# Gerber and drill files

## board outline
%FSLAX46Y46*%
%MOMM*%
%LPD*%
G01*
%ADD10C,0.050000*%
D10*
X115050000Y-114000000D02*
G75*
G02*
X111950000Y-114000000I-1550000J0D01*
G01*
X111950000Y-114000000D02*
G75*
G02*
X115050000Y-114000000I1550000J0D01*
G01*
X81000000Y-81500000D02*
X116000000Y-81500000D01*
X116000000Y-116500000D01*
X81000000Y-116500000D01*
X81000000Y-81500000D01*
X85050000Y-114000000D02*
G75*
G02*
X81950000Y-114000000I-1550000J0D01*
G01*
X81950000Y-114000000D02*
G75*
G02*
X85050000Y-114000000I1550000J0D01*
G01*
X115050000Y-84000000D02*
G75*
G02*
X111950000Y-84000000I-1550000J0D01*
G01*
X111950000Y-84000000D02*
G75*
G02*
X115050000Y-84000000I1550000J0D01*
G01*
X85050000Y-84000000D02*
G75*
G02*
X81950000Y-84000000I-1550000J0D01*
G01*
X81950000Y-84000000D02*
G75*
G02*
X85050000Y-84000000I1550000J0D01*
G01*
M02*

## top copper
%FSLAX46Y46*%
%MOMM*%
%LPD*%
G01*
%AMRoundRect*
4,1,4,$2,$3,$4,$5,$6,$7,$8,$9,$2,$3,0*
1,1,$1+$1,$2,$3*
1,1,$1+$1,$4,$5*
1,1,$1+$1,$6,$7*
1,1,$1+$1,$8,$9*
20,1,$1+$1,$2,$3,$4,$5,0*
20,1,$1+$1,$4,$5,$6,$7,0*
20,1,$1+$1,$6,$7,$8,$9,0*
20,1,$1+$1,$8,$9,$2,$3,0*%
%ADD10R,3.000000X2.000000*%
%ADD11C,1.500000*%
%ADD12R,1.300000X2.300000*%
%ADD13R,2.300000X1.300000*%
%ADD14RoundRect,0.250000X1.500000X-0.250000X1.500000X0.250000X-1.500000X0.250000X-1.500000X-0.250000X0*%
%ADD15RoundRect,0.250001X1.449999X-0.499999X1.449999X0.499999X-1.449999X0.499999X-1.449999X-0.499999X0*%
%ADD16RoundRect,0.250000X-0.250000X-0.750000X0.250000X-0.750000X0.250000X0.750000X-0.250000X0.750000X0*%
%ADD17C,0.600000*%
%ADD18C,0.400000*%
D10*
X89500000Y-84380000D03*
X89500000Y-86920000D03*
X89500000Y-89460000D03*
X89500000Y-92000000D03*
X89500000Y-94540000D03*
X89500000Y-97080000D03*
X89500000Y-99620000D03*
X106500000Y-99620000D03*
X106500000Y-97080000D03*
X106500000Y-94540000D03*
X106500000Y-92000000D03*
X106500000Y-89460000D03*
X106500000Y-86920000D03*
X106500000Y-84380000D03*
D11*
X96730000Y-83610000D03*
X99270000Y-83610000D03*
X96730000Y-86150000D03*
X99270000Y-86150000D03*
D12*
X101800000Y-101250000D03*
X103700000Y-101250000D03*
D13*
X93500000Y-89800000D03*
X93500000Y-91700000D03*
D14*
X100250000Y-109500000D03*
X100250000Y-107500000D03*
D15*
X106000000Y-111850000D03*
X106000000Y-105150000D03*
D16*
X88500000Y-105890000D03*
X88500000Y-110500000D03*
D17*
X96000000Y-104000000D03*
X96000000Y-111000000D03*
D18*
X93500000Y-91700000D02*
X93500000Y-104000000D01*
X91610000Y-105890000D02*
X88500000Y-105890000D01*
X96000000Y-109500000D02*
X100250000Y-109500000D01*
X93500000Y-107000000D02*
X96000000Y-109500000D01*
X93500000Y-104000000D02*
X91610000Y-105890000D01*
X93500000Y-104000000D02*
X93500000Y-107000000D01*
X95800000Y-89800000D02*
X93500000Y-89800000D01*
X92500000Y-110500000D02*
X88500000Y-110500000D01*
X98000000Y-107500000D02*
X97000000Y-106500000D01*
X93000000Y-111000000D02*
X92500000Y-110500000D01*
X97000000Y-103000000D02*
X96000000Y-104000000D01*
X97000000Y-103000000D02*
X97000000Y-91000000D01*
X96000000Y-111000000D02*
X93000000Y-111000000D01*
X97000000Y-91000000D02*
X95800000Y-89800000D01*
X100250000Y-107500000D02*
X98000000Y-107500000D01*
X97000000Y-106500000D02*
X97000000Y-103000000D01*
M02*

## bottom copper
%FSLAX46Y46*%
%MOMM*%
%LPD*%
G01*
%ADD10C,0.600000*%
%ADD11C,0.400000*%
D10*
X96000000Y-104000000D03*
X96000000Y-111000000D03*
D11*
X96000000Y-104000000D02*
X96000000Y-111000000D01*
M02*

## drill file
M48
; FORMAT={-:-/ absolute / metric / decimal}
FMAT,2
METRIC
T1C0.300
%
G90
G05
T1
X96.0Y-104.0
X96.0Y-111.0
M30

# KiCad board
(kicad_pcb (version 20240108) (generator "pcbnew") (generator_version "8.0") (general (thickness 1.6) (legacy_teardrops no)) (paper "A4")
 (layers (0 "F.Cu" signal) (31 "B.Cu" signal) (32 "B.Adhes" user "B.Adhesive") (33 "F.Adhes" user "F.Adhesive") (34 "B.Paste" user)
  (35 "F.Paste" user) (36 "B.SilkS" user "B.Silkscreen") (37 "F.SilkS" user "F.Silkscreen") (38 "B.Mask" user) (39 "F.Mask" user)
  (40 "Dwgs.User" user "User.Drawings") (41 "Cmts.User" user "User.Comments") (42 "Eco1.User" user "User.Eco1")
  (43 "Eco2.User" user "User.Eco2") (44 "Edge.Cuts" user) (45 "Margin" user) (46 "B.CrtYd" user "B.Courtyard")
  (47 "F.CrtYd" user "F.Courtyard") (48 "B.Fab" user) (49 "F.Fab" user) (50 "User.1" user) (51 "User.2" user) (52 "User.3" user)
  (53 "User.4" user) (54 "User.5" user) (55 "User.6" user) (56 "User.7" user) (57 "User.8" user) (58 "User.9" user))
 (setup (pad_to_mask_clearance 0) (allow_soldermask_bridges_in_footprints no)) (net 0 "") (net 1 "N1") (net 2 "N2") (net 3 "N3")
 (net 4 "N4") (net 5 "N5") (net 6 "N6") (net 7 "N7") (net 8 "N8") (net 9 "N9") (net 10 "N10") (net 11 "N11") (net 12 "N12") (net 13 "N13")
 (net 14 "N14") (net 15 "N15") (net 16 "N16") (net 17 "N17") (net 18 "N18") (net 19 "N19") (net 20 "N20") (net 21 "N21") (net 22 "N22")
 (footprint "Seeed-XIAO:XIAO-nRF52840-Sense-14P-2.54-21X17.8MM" (layer "F.Cu") (at 98 92)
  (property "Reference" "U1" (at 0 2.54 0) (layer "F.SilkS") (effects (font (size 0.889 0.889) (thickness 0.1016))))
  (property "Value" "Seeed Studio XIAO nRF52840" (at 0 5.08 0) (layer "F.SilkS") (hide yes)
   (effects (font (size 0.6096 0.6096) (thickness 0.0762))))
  (pad "1" smd rect (at -8.5 -7.62) (size 3 2) (layers "F.Cu" "F.Paste" "F.Mask") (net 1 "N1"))
  (pad "2" smd rect (at -8.5 -5.08) (size 3 2) (layers "F.Cu" "F.Paste" "F.Mask") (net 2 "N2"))
  (pad "3" smd rect (at -8.5 -2.54) (size 3 2) (layers "F.Cu" "F.Paste" "F.Mask") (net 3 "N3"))
  (pad "4" smd rect (at -8.5 0) (size 3 2) (layers "F.Cu" "F.Paste" "F.Mask") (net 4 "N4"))
  (pad "5" smd rect (at -8.5 2.54) (size 3 2) (layers "F.Cu" "F.Paste" "F.Mask") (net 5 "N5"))
  (pad "6" smd rect (at -8.5 5.08 180) (size 3 2) (layers "F.Cu" "F.Paste" "F.Mask") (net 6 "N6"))
  (pad "7" smd rect (at -8.5 7.62) (size 3 2) (layers "F.Cu" "F.Paste" "F.Mask") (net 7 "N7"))
  (pad "8" smd rect (at 8.5 7.62) (size 3 2) (layers "F.Cu" "F.Paste" "F.Mask") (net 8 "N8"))
  (pad "9" smd rect (at 8.5 5.08) (size 3 2) (layers "F.Cu" "F.Paste" "F.Mask") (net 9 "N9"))
  (pad "10" smd rect (at 8.5 2.54) (size 3 2) (layers "F.Cu" "F.Paste" "F.Mask") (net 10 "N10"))
  (pad "11" smd rect (at 8.5 0) (size 3 2) (layers "F.Cu" "F.Paste" "F.Mask") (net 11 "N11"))
  (pad "12" smd rect (at 8.5 -2.54) (size 3 2) (layers "F.Cu" "F.Paste" "F.Mask") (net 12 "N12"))
  (pad "13" smd rect (at 8.5 -5.08) (size 3 2) (layers "F.Cu" "F.Paste" "F.Mask") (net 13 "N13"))
  (pad "14" smd rect (at 8.5 -7.62) (size 3 2) (layers "F.Cu" "F.Paste" "F.Mask") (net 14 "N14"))
  (pad "15" smd circle (at -1.27 -8.39 90) (size 1.5 1.5) (layers "F.Cu" "F.Paste" "F.Mask") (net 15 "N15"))
  (pad "16" smd circle (at 1.27 -8.39 90) (size 1.5 1.5) (layers "F.Cu" "F.Paste" "F.Mask") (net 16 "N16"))
  (pad "17" smd circle (at -1.27 -5.85 90) (size 1.5 1.5) (layers "F.Cu" "F.Paste" "F.Mask") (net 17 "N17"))
  (pad "18" smd circle (at 1.27 -5.85 90) (size 1.5 1.5) (layers "F.Cu" "F.Paste" "F.Mask") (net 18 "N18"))
  (pad "19" smd rect (at 3.8 9.25 90) (size 2.3 1.3) (layers "F.Cu" "F.Paste" "F.Mask") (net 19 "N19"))
  (pad "20" smd rect (at 5.7 9.25 90) (size 2.3 1.3) (layers "F.Cu" "F.Paste" "F.Mask") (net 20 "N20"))
  (pad "21" smd rect (at -4.5 -2.2 180) (size 2.3 1.3) (layers "F.Cu" "F.Paste" "F.Mask") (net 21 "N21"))
  (pad "22" smd rect (at -4.5 -0.3 180) (size 2.3 1.3) (layers "F.Cu" "F.Paste" "F.Mask") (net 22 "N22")))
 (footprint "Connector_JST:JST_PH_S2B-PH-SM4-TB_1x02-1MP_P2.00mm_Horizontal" (layer "F.Cu") (at 103.1 108.5 90)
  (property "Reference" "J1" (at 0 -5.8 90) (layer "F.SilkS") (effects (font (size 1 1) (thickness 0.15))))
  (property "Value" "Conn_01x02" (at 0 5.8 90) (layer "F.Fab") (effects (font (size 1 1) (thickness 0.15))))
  (pad "1" smd roundrect (at -1 -2.85 90) (size 1 3.5) (layers "F.Cu" "F.Paste" "F.Mask") (roundrect_rratio 0.25) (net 22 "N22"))
  (pad "2" smd roundrect (at 1 -2.85 90) (size 1 3.5) (layers "F.Cu" "F.Paste" "F.Mask") (roundrect_rratio 0.25) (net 21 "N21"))
  (pad "MP" smd roundrect (at -3.35 2.9 90) (size 1.5 3.4) (layers "F.Cu" "F.Paste" "F.Mask") (roundrect_rratio 0.166667))
  (pad "MP" smd roundrect (at 3.35 2.9 90) (size 1.5 3.4) (layers "F.Cu" "F.Paste" "F.Mask") (roundrect_rratio 0.166667)))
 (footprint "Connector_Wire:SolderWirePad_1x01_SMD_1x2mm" (layer "F.Cu") (at 88.5 105.89)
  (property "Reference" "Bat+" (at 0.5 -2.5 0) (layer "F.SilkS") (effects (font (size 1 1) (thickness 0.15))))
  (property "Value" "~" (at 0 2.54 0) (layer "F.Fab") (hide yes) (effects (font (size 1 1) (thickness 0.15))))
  (pad "1" smd roundrect (at 0 0) (size 1 2) (layers "F.Cu" "F.Paste" "F.Mask") (roundrect_rratio 0.25) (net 22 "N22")))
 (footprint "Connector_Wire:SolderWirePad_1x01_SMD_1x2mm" (layer "F.Cu") (at 88.5 110.5)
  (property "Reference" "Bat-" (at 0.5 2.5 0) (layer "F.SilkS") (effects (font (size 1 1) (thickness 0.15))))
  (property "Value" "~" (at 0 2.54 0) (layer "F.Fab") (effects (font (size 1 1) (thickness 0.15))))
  (pad "1" smd roundrect (at 0 0) (size 1 2) (layers "F.Cu" "F.Paste" "F.Mask") (roundrect_rratio 0.25) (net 21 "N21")))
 (gr_circle (center 113.5 114) (end 115.05 114) (stroke (width 0.05) (type default)) (fill none) (layer "Edge.Cuts"))
 (gr_rect (start 81 81.5) (end 116 116.5) (stroke (width 0.05) (type default)) (fill none) (layer "Edge.Cuts"))
 (gr_circle (center 83.5 114) (end 85.05 114) (stroke (width 0.05) (type default)) (fill none) (layer "Edge.Cuts"))
 (gr_circle (center 113.5 84) (end 115.05 84) (stroke (width 0.05) (type default)) (fill none) (layer "Edge.Cuts"))
 (gr_circle (center 83.5 84) (end 85.05 84) (stroke (width 0.05) (type default)) (fill none) (layer "Edge.Cuts"))
 (segment (start 93.5 91.7) (end 93.5 104) (width 0.4) (layer "F.Cu") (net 22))
 (segment (start 91.61 105.89) (end 88.5 105.89) (width 0.4) (layer "F.Cu") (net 22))
 (segment (start 96 109.5) (end 100.25 109.5) (width 0.4) (layer "F.Cu") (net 22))
 (segment (start 93.5 107) (end 96 109.5) (width 0.4) (layer "F.Cu") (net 22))
 (segment (start 93.5 104) (end 91.61 105.89) (width 0.4) (layer "F.Cu") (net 22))
 (segment (start 93.5 104) (end 93.5 107) (width 0.4) (layer "F.Cu") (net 22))
 (segment (start 95.8 89.8) (end 93.5 89.8) (width 0.4) (layer "F.Cu") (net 21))
 (segment (start 92.5 110.5) (end 88.5 110.5) (width 0.4) (layer "F.Cu") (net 21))
 (segment (start 98 107.5) (end 97 106.5) (width 0.4) (layer "F.Cu") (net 21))
 (segment (start 93 111) (end 92.5 110.5) (width 0.4) (layer "F.Cu") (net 21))
 (segment (start 97 103) (end 96 104) (width 0.4) (layer "F.Cu") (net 21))
 (segment (start 97 103) (end 97 91) (width 0.4) (layer "F.Cu") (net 21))
 (segment (start 96 111) (end 93 111) (width 0.4) (layer "F.Cu") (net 21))
 (segment (start 97 91) (end 95.8 89.8) (width 0.4) (layer "F.Cu") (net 21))
 (segment (start 100.25 107.5) (end 98 107.5) (width 0.4) (layer "F.Cu") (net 21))
 (segment (start 97 106.5) (end 97 103) (width 0.4) (layer "F.Cu") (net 21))
 (via (at 96 104) (size 0.6) (drill 0.3) (layers "F.Cu" "B.Cu") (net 21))
 (via (at 96 111) (size 0.6) (drill 0.3) (layers "F.Cu" "B.Cu") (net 21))
 (segment (start 96 104) (end 96 111) (width 0.4) (layer "B.Cu") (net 21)))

